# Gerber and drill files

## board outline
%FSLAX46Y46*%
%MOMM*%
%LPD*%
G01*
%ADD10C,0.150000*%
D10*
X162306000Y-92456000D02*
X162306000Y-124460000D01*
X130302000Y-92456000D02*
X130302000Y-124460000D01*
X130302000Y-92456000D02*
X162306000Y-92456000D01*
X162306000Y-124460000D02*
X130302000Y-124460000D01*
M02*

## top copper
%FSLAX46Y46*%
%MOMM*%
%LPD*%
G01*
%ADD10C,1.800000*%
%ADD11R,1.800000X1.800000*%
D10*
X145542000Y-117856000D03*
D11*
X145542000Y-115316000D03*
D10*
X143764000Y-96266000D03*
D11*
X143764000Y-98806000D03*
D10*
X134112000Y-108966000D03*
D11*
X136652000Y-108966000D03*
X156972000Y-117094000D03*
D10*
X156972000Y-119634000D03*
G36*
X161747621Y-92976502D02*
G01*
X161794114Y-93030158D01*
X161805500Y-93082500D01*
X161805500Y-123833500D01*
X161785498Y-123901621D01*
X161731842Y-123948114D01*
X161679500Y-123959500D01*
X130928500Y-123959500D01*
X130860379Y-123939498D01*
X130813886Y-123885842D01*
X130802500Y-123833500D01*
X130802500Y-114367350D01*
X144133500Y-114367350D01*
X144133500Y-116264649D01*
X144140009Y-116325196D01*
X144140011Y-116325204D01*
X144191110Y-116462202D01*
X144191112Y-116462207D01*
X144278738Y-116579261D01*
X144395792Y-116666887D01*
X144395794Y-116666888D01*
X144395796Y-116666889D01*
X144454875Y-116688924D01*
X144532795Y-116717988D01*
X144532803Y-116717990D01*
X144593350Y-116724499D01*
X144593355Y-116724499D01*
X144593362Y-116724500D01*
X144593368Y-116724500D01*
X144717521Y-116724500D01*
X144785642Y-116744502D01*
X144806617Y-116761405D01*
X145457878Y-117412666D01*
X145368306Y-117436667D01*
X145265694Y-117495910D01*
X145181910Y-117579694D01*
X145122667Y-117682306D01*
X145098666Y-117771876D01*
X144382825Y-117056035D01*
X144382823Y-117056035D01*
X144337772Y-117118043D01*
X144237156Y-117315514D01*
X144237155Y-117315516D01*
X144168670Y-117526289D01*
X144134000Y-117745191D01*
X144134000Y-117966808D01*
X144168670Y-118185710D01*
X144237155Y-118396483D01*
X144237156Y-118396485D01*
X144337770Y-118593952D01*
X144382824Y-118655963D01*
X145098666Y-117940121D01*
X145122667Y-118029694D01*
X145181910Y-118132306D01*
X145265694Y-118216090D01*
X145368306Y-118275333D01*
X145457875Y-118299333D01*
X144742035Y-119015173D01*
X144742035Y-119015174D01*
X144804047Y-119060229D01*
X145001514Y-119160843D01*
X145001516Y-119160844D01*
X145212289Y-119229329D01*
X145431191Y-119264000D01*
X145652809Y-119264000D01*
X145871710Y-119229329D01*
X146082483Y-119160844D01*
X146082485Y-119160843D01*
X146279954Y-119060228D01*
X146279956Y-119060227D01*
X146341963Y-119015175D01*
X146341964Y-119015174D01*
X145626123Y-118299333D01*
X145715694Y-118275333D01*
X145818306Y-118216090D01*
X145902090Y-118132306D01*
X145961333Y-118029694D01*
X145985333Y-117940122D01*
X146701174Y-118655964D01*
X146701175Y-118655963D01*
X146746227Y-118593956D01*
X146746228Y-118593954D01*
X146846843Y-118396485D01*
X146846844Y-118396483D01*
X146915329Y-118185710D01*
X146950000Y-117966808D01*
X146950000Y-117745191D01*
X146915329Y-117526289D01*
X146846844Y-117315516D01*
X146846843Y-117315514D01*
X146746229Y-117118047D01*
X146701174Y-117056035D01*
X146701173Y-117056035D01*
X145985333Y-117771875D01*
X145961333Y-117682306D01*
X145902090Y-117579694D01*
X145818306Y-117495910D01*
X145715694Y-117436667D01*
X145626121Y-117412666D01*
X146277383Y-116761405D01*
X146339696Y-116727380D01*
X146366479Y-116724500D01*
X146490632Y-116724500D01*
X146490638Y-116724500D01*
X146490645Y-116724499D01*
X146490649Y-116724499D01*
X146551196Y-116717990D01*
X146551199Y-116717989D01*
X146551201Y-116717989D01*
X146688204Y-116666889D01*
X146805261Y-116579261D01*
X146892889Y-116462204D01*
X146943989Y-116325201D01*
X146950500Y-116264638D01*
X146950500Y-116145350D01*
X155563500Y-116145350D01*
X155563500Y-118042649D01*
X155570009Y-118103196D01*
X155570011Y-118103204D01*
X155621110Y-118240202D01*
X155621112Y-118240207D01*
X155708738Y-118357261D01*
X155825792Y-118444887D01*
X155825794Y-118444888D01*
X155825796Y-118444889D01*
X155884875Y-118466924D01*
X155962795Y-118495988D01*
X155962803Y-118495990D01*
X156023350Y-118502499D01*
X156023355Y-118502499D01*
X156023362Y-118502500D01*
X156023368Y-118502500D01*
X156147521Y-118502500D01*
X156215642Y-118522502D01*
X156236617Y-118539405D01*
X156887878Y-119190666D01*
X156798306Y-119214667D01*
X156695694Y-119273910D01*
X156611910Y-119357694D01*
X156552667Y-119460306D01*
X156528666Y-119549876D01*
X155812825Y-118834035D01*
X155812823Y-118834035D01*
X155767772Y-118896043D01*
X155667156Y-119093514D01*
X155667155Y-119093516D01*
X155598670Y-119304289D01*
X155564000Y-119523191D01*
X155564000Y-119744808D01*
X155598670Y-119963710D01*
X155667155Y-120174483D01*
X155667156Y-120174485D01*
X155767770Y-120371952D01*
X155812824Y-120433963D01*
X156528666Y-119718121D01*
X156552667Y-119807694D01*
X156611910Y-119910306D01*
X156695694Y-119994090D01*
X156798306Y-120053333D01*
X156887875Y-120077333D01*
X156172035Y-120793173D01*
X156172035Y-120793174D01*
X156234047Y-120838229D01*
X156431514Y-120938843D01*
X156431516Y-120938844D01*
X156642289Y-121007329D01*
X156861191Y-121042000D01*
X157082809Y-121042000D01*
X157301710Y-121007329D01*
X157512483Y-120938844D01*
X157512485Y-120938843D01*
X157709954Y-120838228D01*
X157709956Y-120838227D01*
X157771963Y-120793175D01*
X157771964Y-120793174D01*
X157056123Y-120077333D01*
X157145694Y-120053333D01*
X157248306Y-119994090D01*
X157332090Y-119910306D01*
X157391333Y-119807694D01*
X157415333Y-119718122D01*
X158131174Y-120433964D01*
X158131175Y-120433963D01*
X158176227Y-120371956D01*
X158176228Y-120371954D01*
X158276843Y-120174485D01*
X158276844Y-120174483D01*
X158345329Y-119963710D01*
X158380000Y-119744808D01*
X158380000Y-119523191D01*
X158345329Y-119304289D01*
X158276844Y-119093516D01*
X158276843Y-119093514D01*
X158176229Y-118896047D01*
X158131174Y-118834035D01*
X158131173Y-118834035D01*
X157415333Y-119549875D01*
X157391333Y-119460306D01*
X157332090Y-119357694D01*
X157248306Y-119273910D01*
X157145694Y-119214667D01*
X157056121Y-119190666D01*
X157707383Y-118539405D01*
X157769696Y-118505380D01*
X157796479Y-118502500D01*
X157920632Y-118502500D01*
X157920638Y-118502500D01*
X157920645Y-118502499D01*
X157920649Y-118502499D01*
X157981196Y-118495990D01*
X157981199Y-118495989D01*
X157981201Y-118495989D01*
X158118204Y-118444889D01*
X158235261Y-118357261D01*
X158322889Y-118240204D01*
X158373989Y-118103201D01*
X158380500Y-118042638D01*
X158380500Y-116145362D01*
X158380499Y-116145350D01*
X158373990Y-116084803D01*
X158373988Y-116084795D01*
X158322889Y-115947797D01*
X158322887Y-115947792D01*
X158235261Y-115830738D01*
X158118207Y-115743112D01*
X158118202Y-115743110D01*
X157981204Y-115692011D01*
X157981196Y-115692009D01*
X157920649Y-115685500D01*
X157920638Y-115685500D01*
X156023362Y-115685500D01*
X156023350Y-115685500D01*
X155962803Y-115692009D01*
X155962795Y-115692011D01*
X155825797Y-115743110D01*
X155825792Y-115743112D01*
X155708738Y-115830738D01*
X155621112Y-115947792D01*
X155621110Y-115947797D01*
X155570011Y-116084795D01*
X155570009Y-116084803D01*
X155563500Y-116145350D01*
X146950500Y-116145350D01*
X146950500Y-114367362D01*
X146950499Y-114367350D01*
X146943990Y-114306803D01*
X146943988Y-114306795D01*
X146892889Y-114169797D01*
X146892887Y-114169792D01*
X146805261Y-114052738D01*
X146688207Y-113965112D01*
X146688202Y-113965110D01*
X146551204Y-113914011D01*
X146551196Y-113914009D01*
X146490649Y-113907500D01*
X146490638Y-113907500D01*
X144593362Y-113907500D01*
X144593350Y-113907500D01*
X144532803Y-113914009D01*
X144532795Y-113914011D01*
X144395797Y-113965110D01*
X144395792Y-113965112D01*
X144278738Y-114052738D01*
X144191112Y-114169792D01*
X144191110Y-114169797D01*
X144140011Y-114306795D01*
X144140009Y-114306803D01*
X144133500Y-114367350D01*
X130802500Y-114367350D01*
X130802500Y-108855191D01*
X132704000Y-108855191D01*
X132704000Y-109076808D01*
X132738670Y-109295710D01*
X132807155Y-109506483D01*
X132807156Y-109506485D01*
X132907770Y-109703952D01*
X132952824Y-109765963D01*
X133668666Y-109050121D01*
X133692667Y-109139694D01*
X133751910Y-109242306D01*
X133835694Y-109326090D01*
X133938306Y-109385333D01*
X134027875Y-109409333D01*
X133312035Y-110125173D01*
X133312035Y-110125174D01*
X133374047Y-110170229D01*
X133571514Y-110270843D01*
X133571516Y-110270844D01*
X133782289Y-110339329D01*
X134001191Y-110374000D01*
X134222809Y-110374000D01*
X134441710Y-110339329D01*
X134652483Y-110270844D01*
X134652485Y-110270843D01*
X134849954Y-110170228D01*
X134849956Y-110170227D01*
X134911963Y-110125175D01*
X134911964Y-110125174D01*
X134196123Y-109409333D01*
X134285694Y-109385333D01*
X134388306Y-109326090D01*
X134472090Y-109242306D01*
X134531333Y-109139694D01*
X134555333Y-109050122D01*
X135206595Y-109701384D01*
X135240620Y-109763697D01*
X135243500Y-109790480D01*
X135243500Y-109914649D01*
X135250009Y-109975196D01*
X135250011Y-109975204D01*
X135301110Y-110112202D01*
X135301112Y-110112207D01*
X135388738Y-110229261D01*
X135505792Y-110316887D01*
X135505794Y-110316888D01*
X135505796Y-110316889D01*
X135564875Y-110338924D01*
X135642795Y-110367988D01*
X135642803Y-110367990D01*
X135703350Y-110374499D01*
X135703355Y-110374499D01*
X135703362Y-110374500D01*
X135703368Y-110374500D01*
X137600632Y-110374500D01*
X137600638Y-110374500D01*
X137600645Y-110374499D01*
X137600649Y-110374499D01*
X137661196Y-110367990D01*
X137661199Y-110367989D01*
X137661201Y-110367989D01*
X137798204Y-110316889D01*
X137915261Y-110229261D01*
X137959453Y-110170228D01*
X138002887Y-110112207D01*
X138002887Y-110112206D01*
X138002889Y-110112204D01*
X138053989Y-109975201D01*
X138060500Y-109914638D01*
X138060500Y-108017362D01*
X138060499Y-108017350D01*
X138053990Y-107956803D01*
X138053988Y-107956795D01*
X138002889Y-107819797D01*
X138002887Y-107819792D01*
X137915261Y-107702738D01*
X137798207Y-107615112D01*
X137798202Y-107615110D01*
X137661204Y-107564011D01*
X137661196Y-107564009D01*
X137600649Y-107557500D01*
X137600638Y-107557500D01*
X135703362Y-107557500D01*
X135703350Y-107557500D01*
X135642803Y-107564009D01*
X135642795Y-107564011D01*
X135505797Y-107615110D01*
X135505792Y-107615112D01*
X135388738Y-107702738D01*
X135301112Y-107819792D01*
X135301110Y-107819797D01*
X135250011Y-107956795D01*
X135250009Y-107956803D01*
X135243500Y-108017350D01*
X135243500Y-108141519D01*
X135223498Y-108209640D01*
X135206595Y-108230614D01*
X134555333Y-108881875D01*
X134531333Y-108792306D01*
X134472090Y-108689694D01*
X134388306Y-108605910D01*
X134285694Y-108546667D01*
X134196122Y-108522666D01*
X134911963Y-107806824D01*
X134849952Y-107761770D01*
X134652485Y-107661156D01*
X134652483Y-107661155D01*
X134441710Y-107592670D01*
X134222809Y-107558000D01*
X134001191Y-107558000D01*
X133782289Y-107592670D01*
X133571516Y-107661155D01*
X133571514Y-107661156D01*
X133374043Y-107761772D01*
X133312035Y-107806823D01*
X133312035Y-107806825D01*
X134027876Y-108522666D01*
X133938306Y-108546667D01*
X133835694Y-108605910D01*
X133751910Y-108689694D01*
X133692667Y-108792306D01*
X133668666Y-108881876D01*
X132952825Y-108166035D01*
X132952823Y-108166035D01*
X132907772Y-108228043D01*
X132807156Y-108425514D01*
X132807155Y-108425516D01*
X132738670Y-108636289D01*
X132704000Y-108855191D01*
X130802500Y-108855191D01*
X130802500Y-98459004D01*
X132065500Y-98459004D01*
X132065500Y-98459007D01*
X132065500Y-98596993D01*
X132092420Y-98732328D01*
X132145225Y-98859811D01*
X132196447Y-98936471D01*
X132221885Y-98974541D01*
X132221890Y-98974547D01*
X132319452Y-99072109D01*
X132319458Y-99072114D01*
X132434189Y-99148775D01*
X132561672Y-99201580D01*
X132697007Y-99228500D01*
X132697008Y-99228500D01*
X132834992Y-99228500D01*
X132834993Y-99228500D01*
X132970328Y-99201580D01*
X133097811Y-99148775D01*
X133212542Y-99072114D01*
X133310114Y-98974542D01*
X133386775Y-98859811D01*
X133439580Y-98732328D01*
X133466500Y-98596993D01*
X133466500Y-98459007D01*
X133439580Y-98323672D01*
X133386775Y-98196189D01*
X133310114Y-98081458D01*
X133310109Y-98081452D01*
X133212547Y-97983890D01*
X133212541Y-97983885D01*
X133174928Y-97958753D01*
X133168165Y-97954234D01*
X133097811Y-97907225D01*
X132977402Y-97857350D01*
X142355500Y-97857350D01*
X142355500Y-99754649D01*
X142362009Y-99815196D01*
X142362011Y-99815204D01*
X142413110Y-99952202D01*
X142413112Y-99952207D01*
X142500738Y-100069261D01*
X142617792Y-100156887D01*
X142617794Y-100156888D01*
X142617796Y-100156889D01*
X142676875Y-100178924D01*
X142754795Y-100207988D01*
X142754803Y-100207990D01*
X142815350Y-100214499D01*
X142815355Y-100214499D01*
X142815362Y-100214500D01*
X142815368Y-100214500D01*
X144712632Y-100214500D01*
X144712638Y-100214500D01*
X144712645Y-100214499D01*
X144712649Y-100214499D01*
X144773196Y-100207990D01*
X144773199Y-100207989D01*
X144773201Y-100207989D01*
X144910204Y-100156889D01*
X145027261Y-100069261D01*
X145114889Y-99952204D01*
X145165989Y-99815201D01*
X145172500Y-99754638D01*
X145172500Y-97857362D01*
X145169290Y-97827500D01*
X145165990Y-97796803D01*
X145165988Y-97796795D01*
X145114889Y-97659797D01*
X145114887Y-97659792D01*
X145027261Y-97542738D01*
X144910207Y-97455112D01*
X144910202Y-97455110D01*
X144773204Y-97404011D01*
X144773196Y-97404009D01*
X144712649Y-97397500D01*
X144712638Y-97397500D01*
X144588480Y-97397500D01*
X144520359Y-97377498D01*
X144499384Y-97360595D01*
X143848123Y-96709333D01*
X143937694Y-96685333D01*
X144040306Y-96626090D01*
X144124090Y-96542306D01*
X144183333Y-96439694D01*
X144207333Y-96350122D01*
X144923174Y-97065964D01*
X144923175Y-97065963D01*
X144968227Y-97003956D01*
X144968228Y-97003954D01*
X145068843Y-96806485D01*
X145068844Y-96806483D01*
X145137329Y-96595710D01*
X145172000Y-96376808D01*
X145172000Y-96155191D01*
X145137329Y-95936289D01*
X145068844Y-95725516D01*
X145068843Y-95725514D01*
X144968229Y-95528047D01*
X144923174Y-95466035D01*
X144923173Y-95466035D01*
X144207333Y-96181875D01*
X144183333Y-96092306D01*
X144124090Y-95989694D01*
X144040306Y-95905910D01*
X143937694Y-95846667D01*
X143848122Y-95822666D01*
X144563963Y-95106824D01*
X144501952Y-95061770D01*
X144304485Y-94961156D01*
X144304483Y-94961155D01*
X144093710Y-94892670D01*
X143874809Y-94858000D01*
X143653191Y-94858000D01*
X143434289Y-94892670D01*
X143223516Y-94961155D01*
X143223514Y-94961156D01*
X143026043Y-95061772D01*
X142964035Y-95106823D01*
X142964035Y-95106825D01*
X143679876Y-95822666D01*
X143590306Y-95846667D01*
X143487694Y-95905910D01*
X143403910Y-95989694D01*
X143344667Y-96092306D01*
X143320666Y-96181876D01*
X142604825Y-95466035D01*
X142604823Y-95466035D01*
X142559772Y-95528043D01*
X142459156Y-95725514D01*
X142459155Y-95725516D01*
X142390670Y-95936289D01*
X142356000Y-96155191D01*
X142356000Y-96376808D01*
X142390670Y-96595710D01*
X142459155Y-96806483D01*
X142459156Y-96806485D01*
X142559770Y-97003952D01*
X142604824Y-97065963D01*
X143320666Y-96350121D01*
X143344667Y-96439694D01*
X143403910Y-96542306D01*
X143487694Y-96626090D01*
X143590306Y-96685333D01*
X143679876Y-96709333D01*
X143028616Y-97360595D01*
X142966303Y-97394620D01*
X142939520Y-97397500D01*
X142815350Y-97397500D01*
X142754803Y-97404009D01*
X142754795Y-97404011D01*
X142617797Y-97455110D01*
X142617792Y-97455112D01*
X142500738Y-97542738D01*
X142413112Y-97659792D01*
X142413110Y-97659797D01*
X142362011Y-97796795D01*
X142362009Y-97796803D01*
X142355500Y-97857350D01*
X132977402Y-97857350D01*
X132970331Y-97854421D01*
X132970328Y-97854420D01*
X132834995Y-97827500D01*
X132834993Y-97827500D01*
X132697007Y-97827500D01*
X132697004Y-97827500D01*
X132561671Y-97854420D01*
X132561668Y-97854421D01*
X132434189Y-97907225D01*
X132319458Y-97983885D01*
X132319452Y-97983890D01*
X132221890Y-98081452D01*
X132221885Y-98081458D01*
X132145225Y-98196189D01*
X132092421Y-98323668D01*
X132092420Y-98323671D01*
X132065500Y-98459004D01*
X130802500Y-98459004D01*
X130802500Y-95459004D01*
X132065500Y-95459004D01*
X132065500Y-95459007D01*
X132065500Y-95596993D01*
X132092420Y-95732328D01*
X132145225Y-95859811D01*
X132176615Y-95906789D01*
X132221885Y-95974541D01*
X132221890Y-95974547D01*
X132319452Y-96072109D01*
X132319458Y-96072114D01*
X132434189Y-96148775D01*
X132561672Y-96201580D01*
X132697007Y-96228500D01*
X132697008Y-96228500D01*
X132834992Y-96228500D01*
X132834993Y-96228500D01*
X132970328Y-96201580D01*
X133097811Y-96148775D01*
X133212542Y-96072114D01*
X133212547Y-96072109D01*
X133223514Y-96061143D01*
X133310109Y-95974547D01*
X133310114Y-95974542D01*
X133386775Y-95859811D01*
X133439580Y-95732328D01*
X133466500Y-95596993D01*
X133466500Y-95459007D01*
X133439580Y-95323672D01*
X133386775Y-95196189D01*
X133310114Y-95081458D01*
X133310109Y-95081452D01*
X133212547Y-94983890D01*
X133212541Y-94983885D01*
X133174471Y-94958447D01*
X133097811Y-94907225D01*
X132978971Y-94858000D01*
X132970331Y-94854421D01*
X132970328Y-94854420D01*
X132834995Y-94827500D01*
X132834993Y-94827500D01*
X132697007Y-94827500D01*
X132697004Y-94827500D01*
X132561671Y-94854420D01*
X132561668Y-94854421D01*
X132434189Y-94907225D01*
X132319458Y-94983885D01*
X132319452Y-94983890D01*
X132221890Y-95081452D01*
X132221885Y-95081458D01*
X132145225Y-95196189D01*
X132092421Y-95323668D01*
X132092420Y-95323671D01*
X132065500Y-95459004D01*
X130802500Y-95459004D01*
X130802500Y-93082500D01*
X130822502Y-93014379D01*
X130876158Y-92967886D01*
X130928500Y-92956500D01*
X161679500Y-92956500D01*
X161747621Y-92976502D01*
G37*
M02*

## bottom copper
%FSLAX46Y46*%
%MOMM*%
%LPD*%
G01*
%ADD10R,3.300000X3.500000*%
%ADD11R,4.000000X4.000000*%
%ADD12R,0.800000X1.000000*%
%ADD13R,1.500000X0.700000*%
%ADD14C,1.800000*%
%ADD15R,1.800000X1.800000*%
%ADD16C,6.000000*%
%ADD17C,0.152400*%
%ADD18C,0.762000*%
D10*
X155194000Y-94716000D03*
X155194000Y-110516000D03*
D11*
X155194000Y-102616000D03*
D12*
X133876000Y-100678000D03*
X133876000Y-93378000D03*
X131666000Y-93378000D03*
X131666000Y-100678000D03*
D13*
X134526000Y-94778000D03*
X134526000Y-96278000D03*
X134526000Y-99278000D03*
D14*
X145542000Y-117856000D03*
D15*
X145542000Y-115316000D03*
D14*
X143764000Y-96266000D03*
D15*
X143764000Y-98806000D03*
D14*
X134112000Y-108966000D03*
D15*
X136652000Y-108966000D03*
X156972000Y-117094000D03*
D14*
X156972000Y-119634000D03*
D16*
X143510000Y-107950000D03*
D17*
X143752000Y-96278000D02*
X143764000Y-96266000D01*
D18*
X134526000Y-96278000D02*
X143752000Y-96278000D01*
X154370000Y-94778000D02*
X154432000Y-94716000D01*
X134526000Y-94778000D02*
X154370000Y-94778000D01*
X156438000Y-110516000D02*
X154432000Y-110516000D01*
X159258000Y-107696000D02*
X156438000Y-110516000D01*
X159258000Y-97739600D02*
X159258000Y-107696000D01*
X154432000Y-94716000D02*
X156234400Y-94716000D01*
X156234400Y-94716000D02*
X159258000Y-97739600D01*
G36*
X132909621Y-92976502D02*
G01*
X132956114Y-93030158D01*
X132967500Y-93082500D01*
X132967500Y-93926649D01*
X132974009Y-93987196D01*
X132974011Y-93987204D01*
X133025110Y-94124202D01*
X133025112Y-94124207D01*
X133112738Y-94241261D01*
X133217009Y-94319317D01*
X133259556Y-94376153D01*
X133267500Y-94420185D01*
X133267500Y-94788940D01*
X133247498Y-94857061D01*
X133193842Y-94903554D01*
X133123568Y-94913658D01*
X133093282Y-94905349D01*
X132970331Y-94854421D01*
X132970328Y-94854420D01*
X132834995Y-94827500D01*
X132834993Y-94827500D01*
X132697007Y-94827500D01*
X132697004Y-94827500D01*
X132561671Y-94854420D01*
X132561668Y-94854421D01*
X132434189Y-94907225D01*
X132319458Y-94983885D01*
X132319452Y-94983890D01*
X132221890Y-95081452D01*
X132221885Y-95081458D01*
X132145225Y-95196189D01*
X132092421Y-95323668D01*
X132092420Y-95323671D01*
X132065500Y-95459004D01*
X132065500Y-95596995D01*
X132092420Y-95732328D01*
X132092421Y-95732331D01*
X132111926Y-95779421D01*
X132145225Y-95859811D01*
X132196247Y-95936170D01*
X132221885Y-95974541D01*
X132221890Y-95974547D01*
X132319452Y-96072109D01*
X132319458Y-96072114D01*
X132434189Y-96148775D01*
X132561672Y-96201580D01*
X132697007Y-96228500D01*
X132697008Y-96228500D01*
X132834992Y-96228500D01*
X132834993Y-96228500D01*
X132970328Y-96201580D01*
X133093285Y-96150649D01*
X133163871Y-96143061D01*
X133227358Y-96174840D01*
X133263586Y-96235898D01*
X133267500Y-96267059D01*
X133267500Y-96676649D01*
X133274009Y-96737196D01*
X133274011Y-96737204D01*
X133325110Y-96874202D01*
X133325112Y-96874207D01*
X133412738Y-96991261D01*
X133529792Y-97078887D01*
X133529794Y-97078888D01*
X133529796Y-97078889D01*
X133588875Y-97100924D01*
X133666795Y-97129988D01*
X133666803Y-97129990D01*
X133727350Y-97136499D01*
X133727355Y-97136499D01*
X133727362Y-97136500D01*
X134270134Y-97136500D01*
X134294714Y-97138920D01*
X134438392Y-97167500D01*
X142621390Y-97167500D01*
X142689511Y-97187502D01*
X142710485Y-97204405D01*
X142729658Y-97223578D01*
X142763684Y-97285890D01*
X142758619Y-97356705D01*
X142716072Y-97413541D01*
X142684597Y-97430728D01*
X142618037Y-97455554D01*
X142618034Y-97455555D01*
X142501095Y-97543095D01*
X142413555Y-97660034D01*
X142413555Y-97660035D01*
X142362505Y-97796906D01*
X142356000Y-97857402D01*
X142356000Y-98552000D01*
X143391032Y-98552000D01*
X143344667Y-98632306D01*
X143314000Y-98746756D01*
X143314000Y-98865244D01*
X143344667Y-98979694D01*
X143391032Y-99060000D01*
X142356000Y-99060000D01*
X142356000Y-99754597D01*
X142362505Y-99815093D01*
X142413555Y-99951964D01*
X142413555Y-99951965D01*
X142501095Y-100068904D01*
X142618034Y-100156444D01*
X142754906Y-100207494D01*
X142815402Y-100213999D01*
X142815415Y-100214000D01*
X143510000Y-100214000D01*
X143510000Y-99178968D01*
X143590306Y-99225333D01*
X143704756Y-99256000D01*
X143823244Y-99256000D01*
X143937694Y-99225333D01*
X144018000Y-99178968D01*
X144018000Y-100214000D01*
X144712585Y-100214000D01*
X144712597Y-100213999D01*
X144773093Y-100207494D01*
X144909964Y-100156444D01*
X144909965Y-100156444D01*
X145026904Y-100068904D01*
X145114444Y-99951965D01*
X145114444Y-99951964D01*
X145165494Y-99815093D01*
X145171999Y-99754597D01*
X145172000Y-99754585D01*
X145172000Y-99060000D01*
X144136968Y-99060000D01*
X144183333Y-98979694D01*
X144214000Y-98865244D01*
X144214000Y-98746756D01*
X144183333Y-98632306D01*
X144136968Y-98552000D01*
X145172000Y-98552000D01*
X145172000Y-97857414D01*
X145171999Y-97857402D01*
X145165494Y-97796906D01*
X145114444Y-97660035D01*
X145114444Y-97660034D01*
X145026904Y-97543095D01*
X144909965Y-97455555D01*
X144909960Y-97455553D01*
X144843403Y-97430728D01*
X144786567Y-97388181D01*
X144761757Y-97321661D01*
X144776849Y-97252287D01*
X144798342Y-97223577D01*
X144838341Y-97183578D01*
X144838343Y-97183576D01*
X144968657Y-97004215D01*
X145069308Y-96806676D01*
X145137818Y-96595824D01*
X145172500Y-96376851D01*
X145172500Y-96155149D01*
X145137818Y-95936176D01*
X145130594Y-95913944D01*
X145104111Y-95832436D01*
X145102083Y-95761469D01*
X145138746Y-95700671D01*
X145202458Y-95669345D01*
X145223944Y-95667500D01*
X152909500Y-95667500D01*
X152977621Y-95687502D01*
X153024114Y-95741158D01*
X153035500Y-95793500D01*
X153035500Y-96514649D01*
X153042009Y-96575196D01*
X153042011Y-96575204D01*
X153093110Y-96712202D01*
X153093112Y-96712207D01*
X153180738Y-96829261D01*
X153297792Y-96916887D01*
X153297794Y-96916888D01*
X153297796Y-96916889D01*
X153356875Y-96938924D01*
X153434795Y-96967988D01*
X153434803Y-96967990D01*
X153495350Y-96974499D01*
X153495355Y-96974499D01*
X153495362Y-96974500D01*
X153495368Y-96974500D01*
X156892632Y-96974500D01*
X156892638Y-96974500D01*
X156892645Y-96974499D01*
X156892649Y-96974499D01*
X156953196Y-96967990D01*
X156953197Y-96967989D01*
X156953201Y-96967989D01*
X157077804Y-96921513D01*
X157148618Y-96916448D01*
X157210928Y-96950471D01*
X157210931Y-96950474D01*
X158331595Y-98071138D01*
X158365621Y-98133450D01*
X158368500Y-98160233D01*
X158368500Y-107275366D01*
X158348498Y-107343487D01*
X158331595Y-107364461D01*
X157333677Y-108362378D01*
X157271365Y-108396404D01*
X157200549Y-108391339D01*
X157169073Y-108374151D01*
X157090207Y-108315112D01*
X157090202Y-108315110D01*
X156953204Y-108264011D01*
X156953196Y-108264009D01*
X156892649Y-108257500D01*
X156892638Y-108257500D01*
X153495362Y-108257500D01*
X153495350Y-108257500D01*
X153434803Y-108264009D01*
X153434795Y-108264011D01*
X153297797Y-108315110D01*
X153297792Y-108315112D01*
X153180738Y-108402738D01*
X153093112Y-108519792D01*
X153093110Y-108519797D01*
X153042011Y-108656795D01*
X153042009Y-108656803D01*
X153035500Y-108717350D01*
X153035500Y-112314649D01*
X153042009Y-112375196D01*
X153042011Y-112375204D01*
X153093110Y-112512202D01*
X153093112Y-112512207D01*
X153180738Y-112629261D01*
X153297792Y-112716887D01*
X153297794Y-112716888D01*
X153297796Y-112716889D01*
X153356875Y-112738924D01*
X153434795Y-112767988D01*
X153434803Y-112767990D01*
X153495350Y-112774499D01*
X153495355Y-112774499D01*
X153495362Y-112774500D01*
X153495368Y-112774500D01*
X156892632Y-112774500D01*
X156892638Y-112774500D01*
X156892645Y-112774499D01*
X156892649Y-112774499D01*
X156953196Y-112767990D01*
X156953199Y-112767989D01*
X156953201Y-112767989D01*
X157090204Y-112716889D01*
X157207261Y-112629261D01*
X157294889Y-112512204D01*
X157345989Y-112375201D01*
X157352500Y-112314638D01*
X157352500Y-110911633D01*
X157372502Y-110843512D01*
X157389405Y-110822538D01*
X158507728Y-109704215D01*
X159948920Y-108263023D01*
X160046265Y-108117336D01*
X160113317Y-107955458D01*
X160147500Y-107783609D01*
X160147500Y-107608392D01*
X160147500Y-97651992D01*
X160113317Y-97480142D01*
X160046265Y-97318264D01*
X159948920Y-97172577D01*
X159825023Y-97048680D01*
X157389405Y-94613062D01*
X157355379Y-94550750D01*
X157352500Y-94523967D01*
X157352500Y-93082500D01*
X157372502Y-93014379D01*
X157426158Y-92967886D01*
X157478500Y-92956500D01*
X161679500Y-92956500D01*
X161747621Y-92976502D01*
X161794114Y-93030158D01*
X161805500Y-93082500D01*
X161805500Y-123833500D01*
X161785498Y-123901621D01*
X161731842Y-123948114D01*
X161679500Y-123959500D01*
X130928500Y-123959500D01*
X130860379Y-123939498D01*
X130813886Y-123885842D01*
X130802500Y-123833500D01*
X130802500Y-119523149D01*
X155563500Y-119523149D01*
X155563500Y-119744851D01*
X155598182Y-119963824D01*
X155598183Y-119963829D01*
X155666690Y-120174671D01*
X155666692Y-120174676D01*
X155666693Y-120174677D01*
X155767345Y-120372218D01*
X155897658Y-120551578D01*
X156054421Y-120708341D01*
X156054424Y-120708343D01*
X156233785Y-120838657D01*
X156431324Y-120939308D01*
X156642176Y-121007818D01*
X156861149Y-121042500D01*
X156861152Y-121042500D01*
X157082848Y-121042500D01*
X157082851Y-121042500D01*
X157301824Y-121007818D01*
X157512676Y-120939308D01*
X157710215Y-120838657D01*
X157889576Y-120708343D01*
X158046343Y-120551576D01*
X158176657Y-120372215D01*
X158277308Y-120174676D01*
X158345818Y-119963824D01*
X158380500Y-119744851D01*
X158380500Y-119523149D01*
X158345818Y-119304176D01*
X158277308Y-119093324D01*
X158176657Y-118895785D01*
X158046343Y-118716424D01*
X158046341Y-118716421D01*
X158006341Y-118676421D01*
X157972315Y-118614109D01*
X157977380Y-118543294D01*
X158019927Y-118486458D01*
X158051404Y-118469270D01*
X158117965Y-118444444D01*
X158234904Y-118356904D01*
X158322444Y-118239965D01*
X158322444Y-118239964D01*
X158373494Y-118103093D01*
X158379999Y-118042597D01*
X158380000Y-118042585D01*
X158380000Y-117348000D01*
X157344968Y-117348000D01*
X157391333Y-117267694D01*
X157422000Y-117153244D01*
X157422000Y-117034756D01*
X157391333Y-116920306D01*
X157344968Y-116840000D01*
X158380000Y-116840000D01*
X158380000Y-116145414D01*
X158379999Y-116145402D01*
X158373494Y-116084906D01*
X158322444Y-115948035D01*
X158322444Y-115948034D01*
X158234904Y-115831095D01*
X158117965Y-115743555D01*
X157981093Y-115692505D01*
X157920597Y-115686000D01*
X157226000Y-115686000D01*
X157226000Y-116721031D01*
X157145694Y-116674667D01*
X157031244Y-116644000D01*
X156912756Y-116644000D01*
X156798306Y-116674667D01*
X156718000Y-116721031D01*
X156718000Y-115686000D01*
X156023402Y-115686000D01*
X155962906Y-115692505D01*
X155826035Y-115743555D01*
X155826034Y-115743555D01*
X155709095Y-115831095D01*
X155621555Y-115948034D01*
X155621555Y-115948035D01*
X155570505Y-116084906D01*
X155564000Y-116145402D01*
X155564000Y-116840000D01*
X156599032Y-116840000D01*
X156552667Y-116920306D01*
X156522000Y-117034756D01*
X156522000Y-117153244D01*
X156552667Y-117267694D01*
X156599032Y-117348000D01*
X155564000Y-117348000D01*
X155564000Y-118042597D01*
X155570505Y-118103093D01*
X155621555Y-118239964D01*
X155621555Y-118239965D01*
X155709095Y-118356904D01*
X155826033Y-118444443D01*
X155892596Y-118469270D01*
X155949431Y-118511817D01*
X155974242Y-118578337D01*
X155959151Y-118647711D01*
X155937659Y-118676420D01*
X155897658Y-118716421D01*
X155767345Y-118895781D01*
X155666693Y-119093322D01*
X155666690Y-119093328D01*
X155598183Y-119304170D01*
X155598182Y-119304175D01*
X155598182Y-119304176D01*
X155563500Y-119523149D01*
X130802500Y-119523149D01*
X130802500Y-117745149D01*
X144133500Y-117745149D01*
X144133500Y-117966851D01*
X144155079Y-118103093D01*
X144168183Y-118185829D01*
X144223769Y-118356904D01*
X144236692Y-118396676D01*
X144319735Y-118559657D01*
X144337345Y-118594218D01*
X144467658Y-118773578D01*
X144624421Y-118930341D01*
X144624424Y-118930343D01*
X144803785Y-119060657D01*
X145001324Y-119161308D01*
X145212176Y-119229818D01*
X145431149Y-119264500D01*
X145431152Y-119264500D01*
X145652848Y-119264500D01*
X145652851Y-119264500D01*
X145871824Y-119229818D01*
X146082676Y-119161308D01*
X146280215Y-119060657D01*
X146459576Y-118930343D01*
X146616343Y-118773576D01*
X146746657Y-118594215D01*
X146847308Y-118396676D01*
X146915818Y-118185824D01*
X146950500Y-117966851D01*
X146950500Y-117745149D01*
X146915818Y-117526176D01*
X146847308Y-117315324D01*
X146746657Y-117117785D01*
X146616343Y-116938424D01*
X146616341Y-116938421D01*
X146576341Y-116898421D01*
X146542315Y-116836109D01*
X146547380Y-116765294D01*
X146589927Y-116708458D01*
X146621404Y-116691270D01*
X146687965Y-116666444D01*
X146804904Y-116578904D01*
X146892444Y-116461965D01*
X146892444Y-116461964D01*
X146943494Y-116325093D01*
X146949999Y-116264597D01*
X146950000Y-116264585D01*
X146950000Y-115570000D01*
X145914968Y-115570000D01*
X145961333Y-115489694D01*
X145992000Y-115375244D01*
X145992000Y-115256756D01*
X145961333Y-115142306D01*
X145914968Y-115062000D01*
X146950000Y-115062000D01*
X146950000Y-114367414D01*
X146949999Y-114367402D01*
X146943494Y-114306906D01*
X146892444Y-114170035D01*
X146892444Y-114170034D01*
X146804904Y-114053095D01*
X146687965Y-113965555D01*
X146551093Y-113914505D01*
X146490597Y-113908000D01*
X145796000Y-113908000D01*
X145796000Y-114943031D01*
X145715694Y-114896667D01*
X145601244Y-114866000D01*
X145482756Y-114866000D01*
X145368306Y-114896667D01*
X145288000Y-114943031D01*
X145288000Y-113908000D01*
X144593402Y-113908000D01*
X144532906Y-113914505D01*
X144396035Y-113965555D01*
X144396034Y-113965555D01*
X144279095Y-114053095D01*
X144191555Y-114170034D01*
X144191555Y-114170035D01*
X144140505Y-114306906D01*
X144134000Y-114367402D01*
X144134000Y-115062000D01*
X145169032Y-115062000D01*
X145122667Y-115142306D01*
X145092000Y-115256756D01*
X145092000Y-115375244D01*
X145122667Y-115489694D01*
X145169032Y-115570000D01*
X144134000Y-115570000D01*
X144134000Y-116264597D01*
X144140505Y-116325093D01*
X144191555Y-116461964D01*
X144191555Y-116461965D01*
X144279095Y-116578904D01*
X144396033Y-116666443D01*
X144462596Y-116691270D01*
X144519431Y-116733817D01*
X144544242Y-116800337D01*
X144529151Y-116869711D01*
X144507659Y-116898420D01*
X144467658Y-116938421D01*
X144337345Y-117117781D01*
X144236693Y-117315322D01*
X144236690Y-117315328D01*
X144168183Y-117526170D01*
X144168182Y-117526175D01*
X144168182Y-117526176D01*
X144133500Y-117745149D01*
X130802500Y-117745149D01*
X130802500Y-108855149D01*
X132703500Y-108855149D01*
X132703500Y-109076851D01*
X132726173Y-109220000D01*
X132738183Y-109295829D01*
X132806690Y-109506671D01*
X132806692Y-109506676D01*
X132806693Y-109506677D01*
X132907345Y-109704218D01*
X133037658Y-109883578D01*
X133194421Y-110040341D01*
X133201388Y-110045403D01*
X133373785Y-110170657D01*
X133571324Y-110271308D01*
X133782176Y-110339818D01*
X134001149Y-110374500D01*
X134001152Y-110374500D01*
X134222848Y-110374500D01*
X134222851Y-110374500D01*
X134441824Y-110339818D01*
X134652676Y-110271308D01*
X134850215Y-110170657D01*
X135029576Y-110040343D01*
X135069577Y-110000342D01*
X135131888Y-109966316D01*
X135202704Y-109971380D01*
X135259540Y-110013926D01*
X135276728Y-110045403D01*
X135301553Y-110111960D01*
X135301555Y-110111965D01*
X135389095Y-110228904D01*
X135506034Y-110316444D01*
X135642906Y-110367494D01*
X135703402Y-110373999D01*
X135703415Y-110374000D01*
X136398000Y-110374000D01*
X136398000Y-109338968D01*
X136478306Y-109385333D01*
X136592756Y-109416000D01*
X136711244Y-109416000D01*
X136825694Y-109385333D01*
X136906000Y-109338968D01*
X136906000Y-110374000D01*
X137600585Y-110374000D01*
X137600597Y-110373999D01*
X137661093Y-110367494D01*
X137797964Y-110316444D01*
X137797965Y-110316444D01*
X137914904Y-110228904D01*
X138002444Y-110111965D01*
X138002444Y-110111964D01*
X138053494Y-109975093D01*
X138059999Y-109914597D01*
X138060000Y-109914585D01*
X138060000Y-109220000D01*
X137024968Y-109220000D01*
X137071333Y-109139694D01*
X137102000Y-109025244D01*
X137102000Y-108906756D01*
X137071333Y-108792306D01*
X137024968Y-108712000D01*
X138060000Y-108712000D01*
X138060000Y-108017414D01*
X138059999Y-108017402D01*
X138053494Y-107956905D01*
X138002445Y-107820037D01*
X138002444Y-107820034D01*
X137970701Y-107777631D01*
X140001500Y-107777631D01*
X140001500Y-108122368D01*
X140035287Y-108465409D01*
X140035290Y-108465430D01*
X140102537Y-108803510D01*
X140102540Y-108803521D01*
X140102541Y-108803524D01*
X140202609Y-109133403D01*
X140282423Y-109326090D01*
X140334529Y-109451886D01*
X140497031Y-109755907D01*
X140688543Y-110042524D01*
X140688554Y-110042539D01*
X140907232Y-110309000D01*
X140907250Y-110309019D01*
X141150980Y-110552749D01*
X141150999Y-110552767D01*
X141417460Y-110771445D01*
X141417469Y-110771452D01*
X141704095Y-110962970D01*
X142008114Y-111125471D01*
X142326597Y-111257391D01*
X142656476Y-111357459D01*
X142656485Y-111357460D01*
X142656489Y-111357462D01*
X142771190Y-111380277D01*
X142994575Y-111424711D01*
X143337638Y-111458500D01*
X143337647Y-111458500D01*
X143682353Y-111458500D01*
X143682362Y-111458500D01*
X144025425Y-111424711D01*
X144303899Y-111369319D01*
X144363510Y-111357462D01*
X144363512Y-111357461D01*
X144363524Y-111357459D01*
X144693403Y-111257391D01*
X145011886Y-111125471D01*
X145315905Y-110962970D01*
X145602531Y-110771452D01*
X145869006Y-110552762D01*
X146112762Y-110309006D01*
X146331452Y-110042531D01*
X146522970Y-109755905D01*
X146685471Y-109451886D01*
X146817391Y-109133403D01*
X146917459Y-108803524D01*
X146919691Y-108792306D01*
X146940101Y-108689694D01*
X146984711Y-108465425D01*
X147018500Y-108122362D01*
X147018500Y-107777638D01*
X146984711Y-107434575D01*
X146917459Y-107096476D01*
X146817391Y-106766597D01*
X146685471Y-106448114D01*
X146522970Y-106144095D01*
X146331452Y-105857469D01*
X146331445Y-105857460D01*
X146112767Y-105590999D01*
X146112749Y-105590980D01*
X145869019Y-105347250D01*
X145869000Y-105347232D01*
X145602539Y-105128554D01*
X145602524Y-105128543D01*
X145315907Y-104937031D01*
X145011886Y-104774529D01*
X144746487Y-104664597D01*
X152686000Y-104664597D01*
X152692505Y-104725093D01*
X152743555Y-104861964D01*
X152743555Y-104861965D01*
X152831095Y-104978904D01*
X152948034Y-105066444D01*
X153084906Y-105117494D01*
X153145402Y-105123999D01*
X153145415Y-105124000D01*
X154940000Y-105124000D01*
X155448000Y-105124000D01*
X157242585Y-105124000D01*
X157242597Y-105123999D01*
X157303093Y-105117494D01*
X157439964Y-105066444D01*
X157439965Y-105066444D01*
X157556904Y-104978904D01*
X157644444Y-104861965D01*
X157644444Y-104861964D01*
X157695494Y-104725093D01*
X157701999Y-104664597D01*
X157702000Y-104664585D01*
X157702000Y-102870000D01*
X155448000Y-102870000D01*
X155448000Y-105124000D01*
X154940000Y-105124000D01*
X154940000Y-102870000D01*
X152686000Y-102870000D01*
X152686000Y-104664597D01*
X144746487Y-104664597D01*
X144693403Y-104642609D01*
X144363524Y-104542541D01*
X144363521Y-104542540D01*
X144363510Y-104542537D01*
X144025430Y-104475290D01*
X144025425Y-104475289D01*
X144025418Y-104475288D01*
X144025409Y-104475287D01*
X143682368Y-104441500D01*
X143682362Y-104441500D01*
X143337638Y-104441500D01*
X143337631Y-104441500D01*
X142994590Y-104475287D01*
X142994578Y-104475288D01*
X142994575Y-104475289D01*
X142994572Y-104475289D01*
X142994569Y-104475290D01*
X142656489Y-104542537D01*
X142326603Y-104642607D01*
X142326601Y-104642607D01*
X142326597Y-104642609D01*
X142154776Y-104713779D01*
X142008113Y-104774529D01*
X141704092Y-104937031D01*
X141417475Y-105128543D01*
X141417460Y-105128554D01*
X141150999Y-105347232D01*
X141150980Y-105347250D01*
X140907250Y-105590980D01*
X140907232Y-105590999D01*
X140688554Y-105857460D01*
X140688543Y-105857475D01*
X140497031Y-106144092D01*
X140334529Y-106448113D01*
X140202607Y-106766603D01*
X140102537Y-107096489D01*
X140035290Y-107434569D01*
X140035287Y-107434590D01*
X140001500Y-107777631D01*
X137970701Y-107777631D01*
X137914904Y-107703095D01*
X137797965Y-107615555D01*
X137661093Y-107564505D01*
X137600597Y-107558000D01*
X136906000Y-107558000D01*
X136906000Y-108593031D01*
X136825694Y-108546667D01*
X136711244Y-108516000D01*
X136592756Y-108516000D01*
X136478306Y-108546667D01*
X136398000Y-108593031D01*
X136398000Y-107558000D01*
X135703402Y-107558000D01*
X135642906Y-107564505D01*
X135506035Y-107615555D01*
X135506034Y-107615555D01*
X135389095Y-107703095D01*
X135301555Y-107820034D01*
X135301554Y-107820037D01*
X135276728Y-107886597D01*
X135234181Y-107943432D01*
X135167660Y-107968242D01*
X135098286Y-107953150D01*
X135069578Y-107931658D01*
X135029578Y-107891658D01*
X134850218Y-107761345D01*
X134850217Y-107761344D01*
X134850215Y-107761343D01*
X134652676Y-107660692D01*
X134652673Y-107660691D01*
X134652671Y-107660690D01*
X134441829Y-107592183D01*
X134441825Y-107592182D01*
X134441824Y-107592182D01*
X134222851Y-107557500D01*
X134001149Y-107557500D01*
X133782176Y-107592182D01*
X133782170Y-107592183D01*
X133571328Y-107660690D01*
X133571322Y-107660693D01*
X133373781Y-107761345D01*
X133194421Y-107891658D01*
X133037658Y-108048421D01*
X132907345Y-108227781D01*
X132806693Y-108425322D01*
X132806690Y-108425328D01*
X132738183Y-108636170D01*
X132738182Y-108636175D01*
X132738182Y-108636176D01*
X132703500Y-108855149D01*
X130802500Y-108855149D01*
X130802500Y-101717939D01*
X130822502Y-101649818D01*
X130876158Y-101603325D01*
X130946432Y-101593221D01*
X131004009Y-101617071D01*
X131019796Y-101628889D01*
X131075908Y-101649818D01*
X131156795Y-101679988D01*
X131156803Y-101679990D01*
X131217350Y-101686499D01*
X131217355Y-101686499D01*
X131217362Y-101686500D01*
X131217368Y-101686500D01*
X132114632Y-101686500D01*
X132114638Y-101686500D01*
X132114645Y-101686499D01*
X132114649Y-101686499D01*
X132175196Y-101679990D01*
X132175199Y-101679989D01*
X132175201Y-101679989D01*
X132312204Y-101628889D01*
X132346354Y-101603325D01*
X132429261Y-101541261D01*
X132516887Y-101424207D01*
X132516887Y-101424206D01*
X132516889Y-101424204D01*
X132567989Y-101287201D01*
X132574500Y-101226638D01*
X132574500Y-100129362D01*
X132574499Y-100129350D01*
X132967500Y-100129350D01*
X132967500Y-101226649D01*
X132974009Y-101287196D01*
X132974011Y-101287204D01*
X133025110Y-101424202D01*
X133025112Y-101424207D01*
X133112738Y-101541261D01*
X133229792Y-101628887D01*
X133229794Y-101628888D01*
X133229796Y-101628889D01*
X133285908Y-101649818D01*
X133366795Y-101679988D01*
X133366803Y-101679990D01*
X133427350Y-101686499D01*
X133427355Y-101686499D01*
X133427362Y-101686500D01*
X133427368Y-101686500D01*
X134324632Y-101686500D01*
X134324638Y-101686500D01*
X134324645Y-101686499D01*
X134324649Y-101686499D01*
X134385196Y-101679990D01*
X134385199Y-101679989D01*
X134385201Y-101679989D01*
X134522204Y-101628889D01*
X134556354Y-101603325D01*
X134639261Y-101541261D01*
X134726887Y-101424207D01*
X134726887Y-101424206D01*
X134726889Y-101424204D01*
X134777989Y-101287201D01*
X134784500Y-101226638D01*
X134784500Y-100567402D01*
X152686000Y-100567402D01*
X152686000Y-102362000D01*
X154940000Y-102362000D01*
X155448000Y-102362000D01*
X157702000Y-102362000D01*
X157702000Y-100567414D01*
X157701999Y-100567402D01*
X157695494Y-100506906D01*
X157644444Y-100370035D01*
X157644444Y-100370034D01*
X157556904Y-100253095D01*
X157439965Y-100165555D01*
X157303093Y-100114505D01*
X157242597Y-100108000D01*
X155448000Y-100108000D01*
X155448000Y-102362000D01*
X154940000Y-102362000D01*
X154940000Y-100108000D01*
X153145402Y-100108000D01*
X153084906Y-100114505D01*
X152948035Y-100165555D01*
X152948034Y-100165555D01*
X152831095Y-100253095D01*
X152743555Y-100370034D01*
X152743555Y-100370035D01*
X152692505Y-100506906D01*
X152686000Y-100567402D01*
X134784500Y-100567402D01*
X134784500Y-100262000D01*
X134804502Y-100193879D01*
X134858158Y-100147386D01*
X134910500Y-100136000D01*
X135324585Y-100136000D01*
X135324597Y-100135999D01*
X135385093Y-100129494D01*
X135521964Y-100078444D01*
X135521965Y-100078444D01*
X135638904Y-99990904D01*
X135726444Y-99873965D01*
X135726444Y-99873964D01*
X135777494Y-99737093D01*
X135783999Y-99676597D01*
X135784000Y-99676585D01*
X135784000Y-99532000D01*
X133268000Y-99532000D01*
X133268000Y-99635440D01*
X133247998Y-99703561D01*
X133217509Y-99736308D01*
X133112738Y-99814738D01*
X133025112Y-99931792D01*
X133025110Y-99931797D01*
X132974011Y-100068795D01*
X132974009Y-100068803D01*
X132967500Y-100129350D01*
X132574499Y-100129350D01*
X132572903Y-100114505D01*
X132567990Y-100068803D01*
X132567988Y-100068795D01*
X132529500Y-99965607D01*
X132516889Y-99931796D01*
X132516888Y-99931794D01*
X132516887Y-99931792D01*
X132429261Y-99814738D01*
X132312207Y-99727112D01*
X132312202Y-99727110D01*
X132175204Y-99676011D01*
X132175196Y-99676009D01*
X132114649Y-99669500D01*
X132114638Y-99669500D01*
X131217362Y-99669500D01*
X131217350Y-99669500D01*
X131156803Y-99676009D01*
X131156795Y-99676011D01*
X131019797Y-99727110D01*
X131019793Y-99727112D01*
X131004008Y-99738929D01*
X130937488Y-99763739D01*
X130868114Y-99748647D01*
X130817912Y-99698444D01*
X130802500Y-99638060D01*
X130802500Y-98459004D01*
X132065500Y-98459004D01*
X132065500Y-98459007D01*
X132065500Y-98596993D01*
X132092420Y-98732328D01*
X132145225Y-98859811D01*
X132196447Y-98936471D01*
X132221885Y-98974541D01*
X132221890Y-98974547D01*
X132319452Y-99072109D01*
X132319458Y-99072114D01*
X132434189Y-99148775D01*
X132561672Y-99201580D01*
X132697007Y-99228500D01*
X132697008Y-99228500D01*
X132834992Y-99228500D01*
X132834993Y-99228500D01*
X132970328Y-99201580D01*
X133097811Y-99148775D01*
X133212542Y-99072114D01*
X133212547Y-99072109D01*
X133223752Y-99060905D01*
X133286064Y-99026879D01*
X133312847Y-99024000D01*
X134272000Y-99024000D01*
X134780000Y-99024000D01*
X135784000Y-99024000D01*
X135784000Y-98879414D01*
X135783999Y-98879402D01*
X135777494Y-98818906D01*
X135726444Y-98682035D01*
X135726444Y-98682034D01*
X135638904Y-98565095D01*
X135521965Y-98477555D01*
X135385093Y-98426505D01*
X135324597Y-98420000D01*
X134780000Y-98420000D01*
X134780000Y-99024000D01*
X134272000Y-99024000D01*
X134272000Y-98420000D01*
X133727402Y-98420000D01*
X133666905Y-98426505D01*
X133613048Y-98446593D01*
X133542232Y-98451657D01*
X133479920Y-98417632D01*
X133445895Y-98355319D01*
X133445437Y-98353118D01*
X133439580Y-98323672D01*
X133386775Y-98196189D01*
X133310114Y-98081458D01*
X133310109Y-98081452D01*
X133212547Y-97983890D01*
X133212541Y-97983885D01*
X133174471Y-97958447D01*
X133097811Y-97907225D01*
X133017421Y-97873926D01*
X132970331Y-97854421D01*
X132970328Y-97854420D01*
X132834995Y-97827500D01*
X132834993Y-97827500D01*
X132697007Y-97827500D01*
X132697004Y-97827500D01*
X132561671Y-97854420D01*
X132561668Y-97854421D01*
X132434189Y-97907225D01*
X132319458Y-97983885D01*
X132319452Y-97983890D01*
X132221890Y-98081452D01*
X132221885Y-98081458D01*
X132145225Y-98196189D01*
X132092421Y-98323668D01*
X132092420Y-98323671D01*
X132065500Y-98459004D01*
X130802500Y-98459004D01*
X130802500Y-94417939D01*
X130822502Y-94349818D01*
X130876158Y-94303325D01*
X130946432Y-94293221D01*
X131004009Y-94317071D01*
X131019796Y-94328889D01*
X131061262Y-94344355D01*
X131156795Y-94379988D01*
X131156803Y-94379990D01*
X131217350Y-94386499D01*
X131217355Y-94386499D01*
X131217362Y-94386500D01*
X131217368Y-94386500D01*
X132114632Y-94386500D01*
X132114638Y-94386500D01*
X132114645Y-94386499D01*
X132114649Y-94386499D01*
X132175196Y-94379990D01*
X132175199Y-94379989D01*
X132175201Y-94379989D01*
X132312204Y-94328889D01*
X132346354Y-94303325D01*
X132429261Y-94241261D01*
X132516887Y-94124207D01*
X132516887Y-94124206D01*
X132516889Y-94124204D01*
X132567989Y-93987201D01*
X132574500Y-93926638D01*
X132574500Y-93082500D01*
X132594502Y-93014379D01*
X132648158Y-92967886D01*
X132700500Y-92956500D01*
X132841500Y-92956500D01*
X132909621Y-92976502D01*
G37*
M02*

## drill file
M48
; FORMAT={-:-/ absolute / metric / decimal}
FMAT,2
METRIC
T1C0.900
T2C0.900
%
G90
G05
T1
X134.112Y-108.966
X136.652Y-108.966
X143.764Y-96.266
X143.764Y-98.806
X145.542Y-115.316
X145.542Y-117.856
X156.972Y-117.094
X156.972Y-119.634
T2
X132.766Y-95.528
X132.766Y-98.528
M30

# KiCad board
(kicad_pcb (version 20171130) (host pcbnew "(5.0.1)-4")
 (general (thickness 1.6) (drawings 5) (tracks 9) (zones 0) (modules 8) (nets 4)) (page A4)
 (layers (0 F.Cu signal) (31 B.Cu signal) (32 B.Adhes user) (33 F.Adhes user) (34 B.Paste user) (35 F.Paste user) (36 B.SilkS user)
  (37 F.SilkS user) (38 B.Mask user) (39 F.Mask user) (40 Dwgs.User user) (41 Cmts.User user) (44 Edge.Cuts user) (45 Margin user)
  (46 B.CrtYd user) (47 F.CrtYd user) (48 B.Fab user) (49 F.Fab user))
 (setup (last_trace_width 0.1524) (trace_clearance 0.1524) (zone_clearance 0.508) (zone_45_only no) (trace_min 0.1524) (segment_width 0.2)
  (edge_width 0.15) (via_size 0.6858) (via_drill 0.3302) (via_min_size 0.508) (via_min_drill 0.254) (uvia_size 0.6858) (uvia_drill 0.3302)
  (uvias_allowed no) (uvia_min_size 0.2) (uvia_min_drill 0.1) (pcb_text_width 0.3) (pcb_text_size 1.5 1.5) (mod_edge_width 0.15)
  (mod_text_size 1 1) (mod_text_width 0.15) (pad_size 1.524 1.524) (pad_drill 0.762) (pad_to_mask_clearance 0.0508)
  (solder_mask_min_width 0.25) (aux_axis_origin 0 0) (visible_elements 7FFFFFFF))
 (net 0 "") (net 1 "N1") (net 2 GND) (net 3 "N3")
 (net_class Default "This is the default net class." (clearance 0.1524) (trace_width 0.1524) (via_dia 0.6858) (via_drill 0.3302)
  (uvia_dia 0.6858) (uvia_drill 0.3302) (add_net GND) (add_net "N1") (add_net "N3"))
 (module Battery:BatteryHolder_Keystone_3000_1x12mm (layer B.Cu) (at 155.194 102.616 270)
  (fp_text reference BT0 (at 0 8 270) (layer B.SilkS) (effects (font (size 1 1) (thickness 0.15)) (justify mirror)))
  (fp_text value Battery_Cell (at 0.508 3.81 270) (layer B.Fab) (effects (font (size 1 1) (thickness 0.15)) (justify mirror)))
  (pad 1 smd rect (at -7.9 0 270) (size 3.5 3.3) (layers B.Cu B.Paste B.Mask) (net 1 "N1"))
  (pad 1 smd rect (at 7.9 0 270) (size 3.5 3.3) (layers B.Cu B.Paste B.Mask) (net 1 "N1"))
  (pad 2 smd rect (at 0 0 270) (size 4 4) (layers B.Cu B.Mask) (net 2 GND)))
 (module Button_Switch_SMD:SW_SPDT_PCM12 (layer B.Cu) (at 133.096 97.028 90)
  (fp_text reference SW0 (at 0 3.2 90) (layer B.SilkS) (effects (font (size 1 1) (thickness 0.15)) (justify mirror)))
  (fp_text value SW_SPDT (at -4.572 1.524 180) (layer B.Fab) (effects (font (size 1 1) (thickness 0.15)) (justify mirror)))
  (pad "" smd rect (at -3.65 0.78 90) (size 1 0.8) (layers B.Cu B.Paste B.Mask))
  (pad "" smd rect (at 3.65 0.78 90) (size 1 0.8) (layers B.Cu B.Paste B.Mask))
  (pad "" smd rect (at 3.65 -1.43 90) (size 1 0.8) (layers B.Cu B.Paste B.Mask))
  (pad "" smd rect (at -3.65 -1.43 90) (size 1 0.8) (layers B.Cu B.Paste B.Mask))
  (pad 3 smd rect (at 2.25 1.43 90) (size 0.7 1.5) (layers B.Cu B.Paste B.Mask) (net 1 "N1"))
  (pad 2 smd rect (at 0.75 1.43 90) (size 0.7 1.5) (layers B.Cu B.Paste B.Mask) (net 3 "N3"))
  (pad 1 smd rect (at -2.25 1.43 90) (size 0.7 1.5) (layers B.Cu B.Paste B.Mask) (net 2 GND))
  (pad "" np_thru_hole circle (at 1.5 -0.33 90) (size 0.9 0.9) (drill 0.9) (layers *.Cu *.Mask))
  (pad "" np_thru_hole circle (at -1.5 -0.33 90) (size 0.9 0.9) (drill 0.9) (layers *.Cu *.Mask)))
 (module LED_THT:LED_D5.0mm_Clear (layer F.Cu) (at 145.542 115.316 270)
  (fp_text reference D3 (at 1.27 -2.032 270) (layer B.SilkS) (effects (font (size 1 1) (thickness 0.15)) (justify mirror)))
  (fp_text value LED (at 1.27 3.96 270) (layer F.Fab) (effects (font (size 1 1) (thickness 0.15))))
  (pad 2 thru_hole circle (at 2.54 0 270) (size 1.8 1.8) (drill 0.9) (layers *.Cu *.Mask) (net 3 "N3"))
  (pad 1 thru_hole rect (at 0 0 270) (size 1.8 1.8) (drill 0.9) (layers *.Cu *.Mask) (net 2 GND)))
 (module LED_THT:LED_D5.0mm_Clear (layer F.Cu) (at 143.764 98.806 90)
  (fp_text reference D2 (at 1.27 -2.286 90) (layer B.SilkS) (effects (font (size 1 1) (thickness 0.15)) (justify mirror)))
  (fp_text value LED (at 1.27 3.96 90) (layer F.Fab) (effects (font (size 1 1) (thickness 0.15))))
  (pad 2 thru_hole circle (at 2.54 0 90) (size 1.8 1.8) (drill 0.9) (layers *.Cu *.Mask) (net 3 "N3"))
  (pad 1 thru_hole rect (at 0 0 90) (size 1.8 1.8) (drill 0.9) (layers *.Cu *.Mask) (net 2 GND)))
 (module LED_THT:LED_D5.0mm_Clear (layer F.Cu) (at 136.652 108.966 180)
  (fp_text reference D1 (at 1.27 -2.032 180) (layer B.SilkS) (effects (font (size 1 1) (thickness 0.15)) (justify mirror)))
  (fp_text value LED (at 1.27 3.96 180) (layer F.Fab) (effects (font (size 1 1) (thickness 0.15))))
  (pad 2 thru_hole circle (at 2.54 0 180) (size 1.8 1.8) (drill 0.9) (layers *.Cu *.Mask) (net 3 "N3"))
  (pad 1 thru_hole rect (at 0 0 180) (size 1.8 1.8) (drill 0.9) (layers *.Cu *.Mask) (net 2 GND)))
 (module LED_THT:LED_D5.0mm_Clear (layer F.Cu) (at 156.972 117.094 270)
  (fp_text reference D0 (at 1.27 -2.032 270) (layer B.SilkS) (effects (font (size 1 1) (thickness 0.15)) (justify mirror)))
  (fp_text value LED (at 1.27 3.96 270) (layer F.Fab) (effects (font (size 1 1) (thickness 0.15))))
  (pad 1 thru_hole rect (at 0 0 270) (size 1.8 1.8) (drill 0.9) (layers *.Cu *.Mask) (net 2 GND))
  (pad 2 thru_hole circle (at 2.54 0 270) (size 1.8 1.8) (drill 0.9) (layers *.Cu *.Mask) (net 3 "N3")))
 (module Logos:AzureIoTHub (layer F.Cu) (at 146.304 108.458)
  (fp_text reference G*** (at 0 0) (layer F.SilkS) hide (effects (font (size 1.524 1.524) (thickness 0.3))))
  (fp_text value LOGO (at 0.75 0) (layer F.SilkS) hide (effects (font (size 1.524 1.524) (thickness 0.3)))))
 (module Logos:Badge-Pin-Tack (layer B.Cu) (at 143.51 107.95)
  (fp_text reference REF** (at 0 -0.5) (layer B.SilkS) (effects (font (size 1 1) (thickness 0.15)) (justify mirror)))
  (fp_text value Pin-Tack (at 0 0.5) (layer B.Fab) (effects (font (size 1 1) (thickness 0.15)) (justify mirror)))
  (pad 1 smd circle (at 0 0) (size 6 6) (layers B.Cu B.Paste B.Mask)))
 (gr_line (start 162.306 92.456) (end 162.306 124.46) (layer Edge.Cuts) (width 0.15))
 (gr_line (start 130.302 92.456) (end 130.302 124.46) (layer Edge.Cuts) (width 0.15))
 (gr_line (start 130.302 92.456) (end 162.306 92.456) (layer Edge.Cuts) (width 0.15))
 (gr_line (start 162.306 124.46) (end 130.302 124.46) (layer Edge.Cuts) (width 0.15))
 (segment (start 143.752 96.278) (end 143.764 96.266) (width 0.1524) (layer B.Cu) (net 3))
 (segment (start 134.526 96.278) (end 143.752 96.278) (width 0.762) (layer B.Cu) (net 3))
 (segment (start 154.37 94.778) (end 154.432 94.716) (width 0.762) (layer B.Cu) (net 1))
 (segment (start 134.526 94.778) (end 154.37 94.778) (width 0.762) (layer B.Cu) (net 1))
 (segment (start 156.438 110.516) (end 154.432 110.516) (width 0.762) (layer B.Cu) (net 1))
 (segment (start 159.258 107.696) (end 156.438 110.516) (width 0.762) (layer B.Cu) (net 1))
 (segment (start 159.258 97.7396) (end 159.258 107.696) (width 0.762) (layer B.Cu) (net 1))
 (segment (start 154.432 94.716) (end 156.2344 94.716) (width 0.762) (layer B.Cu) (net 1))
 (segment (start 156.2344 94.716) (end 159.258 97.7396) (width 0.762) (layer B.Cu) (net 1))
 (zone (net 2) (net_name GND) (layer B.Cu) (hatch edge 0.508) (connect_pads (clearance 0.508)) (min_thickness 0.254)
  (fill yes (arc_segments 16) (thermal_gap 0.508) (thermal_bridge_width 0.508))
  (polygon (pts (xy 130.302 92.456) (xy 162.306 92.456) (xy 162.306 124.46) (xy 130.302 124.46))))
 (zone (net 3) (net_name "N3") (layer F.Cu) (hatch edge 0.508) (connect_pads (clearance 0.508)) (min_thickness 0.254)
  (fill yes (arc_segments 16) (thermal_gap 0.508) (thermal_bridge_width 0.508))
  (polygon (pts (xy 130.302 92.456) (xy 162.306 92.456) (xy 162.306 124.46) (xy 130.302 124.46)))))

